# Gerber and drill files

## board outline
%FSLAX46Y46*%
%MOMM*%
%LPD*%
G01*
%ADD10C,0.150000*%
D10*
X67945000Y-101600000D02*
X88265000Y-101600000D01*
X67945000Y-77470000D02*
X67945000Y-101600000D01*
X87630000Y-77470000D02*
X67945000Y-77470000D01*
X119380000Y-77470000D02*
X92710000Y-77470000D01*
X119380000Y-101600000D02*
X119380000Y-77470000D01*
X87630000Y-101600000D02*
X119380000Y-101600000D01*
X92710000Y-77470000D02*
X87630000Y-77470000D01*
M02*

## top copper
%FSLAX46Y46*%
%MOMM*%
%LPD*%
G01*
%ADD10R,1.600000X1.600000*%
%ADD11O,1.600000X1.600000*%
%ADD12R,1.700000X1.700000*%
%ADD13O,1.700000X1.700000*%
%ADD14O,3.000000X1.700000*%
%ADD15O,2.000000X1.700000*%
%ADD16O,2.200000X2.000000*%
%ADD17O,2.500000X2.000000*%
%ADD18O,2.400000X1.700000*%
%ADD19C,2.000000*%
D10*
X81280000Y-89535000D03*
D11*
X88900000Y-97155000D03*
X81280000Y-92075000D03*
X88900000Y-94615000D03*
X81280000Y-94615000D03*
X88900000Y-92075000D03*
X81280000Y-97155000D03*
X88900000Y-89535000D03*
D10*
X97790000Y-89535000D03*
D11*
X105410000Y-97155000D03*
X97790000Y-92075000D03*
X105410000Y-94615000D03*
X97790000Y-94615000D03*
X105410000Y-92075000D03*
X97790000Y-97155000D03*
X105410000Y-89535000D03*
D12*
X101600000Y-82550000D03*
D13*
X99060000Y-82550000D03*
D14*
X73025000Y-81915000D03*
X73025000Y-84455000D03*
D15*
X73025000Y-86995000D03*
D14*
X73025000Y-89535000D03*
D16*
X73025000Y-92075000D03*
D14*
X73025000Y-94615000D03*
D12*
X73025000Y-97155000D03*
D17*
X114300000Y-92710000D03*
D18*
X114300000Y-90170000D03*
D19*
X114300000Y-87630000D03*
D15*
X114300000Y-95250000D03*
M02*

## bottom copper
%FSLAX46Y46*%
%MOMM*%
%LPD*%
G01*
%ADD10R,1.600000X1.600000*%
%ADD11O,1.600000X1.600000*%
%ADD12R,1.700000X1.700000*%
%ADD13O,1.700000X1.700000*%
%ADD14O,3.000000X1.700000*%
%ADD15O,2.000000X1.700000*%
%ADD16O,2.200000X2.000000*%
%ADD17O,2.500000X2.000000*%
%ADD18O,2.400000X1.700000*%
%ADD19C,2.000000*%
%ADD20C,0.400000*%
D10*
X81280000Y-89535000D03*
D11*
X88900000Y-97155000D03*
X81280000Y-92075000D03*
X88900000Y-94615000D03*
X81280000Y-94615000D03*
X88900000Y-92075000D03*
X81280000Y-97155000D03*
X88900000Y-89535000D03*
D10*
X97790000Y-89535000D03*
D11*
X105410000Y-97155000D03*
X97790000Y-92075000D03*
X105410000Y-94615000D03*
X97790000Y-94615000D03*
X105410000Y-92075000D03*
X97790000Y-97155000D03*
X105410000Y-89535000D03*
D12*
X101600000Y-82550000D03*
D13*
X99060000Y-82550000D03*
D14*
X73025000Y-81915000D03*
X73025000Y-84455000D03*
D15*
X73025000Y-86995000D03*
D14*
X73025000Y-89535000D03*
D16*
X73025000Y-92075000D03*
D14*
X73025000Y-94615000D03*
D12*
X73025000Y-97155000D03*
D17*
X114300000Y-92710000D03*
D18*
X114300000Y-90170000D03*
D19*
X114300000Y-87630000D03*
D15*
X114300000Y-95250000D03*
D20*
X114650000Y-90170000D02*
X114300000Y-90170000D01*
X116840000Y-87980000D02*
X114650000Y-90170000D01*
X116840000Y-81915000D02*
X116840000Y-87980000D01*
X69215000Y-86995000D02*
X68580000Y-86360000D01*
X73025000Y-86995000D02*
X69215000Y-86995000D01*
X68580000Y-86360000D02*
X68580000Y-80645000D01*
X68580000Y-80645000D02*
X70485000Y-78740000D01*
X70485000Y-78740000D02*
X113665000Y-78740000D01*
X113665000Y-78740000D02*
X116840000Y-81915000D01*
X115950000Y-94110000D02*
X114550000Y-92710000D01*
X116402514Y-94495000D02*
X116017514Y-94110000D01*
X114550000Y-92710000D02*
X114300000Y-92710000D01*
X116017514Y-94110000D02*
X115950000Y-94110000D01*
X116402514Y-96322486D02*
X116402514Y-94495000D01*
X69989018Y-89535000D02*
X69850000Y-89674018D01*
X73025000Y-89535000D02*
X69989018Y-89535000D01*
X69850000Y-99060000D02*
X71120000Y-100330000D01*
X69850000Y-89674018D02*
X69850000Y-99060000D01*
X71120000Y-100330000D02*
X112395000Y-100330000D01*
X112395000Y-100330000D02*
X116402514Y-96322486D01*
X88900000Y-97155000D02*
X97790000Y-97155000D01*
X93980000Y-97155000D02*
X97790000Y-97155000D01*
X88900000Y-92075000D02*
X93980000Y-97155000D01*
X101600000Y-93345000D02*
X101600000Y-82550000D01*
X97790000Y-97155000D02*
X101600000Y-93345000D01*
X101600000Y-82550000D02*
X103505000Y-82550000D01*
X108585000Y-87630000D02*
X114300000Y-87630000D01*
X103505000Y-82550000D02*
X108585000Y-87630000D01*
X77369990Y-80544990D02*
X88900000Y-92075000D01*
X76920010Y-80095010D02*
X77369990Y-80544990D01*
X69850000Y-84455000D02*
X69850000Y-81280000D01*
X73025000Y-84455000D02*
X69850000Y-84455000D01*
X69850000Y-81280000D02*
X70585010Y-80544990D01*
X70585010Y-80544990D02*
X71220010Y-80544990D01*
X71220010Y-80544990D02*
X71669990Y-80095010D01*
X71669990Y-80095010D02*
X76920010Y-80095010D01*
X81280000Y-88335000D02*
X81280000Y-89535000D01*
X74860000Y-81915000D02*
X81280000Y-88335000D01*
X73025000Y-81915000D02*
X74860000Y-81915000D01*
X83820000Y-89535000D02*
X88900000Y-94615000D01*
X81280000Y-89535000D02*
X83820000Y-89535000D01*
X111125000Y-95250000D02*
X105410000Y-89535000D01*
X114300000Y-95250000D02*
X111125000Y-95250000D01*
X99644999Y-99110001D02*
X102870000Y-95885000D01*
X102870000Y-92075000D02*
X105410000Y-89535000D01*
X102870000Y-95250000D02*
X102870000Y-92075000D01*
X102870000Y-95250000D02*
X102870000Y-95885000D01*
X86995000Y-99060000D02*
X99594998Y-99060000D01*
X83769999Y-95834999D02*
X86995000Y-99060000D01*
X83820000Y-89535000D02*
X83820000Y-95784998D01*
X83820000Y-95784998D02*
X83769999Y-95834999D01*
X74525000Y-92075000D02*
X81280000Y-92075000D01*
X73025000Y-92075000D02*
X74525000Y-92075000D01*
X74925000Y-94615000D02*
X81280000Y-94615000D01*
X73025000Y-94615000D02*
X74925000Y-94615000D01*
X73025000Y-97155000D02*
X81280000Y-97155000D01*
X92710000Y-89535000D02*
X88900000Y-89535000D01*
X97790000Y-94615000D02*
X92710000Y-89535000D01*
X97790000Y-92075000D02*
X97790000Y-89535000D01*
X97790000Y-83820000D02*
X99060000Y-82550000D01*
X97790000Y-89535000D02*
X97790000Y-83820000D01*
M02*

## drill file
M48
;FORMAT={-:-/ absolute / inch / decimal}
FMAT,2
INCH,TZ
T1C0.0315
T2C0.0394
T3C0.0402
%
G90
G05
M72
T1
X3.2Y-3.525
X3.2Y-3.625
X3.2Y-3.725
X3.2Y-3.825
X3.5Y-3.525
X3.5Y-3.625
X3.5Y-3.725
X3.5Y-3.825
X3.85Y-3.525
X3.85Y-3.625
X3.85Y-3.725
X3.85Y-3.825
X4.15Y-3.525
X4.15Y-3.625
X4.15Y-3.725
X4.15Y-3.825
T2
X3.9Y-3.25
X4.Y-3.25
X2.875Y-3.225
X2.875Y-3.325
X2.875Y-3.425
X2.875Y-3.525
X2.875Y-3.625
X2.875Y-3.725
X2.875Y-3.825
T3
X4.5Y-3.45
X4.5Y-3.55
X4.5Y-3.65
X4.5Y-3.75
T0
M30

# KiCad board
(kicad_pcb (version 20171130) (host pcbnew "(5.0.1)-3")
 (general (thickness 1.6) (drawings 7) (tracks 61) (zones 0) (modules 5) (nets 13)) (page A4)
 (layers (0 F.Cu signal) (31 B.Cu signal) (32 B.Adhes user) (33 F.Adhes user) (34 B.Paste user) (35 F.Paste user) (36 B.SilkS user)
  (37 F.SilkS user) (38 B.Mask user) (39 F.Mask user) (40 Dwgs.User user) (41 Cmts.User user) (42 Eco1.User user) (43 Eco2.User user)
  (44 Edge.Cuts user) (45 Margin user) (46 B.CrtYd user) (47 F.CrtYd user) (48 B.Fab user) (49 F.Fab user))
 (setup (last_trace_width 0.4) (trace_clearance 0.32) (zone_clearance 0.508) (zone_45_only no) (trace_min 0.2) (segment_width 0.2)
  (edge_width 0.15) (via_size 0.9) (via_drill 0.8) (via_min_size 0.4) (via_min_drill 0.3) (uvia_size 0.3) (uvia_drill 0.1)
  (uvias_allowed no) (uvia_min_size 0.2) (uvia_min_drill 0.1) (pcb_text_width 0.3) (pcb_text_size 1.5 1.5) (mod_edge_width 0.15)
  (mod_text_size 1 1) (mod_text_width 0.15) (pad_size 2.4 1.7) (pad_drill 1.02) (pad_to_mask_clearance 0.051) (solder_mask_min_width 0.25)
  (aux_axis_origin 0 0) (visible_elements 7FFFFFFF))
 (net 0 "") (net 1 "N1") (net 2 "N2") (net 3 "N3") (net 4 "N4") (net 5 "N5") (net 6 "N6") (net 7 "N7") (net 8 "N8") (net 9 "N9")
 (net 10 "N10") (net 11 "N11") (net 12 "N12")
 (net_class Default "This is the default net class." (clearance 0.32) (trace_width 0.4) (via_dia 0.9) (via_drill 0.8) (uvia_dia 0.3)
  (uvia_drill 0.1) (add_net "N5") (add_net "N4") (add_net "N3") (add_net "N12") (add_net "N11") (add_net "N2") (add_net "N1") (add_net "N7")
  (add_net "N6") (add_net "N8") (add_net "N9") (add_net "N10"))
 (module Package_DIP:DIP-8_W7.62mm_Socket (layer F.Cu) (at 81.28 89.535)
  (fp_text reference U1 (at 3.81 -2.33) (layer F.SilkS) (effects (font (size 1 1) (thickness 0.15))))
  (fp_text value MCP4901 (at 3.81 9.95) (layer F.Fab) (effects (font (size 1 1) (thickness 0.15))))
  (pad 1 thru_hole rect (at 0 0) (size 1.6 1.6) (drill 0.8) (layers *.Cu *.Mask) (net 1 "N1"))
  (pad 5 thru_hole oval (at 7.62 7.62) (size 1.6 1.6) (drill 0.8) (layers *.Cu *.Mask) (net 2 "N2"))
  (pad 2 thru_hole oval (at 0 2.54) (size 1.6 1.6) (drill 0.8) (layers *.Cu *.Mask) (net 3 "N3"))
  (pad 6 thru_hole oval (at 7.62 5.08) (size 1.6 1.6) (drill 0.8) (layers *.Cu *.Mask) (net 1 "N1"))
  (pad 3 thru_hole oval (at 0 5.08) (size 1.6 1.6) (drill 0.8) (layers *.Cu *.Mask) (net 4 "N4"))
  (pad 7 thru_hole oval (at 7.62 2.54) (size 1.6 1.6) (drill 0.8) (layers *.Cu *.Mask) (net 2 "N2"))
  (pad 4 thru_hole oval (at 0 7.62) (size 1.6 1.6) (drill 0.8) (layers *.Cu *.Mask) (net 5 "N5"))
  (pad 8 thru_hole oval (at 7.62 0) (size 1.6 1.6) (drill 0.8) (layers *.Cu *.Mask) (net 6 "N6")))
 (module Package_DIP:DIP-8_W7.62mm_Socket (layer F.Cu) (at 97.79 89.535)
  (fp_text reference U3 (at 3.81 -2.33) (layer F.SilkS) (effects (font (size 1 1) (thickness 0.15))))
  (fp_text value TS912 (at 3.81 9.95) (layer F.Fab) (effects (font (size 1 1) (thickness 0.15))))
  (pad 1 thru_hole rect (at 0 0) (size 1.6 1.6) (drill 0.8) (layers *.Cu *.Mask) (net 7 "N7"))
  (pad 5 thru_hole oval (at 7.62 7.62) (size 1.6 1.6) (drill 0.8) (layers *.Cu *.Mask) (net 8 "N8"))
  (pad 2 thru_hole oval (at 0 2.54) (size 1.6 1.6) (drill 0.8) (layers *.Cu *.Mask) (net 7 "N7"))
  (pad 6 thru_hole oval (at 7.62 5.08) (size 1.6 1.6) (drill 0.8) (layers *.Cu *.Mask) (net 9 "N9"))
  (pad 3 thru_hole oval (at 0 5.08) (size 1.6 1.6) (drill 0.8) (layers *.Cu *.Mask) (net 6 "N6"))
  (pad 7 thru_hole oval (at 7.62 2.54) (size 1.6 1.6) (drill 0.8) (layers *.Cu *.Mask) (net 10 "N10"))
  (pad 4 thru_hole oval (at 0 7.62) (size 1.6 1.6) (drill 0.8) (layers *.Cu *.Mask) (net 2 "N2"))
  (pad 8 thru_hole oval (at 7.62 0) (size 1.6 1.6) (drill 0.8) (layers *.Cu *.Mask) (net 1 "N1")))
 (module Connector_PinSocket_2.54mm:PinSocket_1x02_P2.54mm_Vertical (layer F.Cu) (at 101.6 82.55 270)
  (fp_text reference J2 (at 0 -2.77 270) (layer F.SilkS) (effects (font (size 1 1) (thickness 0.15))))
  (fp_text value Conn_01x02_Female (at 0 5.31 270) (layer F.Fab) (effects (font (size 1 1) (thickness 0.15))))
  (pad 1 thru_hole rect (at 0 0 270) (size 1.7 1.7) (drill 1) (layers *.Cu *.Mask) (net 2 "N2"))
  (pad 2 thru_hole oval (at 0 2.54 270) (size 1.7 1.7) (drill 1) (layers *.Cu *.Mask) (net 7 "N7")))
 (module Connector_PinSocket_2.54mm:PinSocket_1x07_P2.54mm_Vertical (layer F.Cu) (at 73.025 97.155 180)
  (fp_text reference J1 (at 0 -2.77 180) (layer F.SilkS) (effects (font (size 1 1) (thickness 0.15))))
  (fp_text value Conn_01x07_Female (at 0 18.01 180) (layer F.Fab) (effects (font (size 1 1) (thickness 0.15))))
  (pad 7 thru_hole oval (at 0 15.24 180) (size 3 1.7) (drill 1) (layers *.Cu *.Mask) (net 1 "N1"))
  (pad 6 thru_hole oval (at 0 12.7 180) (size 3 1.7) (drill 1) (layers *.Cu *.Mask) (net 2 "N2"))
  (pad 5 thru_hole oval (at 0 10.16 180) (size 2 1.7) (drill 1) (layers *.Cu *.Mask) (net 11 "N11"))
  (pad 4 thru_hole oval (at 0 7.62 180) (size 3 1.7) (drill 1) (layers *.Cu *.Mask) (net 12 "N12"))
  (pad 3 thru_hole oval (at 0 5.08 180) (size 2.2 2) (drill 1) (layers *.Cu *.Mask) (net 3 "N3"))
  (pad 2 thru_hole oval (at 0 2.54 180) (size 3 1.7) (drill 1) (layers *.Cu *.Mask) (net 4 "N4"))
  (pad 1 thru_hole rect (at 0 0 180) (size 1.7 1.7) (drill 1) (layers *.Cu *.Mask) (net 5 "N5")))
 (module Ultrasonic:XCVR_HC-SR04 (layer F.Cu) (at 114.3 91.44 90)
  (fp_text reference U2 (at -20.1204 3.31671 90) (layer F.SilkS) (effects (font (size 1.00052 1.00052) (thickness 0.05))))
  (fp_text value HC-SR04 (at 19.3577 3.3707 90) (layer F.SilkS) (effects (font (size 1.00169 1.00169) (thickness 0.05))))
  (pad 2 thru_hole oval (at -1.27 0 90) (size 2 2.5) (drill 1.02) (layers *.Cu *.Mask) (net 12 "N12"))
  (pad 3 thru_hole oval (at 1.27 0 180) (size 2.4 1.7) (drill 1.02) (layers *.Cu *.Mask) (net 11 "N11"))
  (pad 4 thru_hole circle (at 3.81 0 90) (size 2 2) (drill 1.02) (layers *.Cu *.Mask) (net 2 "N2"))
  (pad 1 thru_hole oval (at -3.81 0 180) (size 2 1.7) (drill 1.02) (layers *.Cu *.Mask) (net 1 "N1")))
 (gr_line (start 67.945 101.6) (end 88.265 101.6) (layer Edge.Cuts) (width 0.15))
 (gr_line (start 67.945 77.47) (end 67.945 101.6) (layer Edge.Cuts) (width 0.15))
 (gr_line (start 87.63 77.47) (end 67.945 77.47) (layer Edge.Cuts) (width 0.15))
 (gr_line (start 119.38 77.47) (end 92.71 77.47) (layer Edge.Cuts) (width 0.15))
 (gr_line (start 119.38 101.6) (end 119.38 77.47) (layer Edge.Cuts) (width 0.15))
 (gr_line (start 87.63 101.6) (end 119.38 101.6) (layer Edge.Cuts) (width 0.15))
 (gr_line (start 92.71 77.47) (end 87.63 77.47) (layer Edge.Cuts) (width 0.15))
 (segment (start 114.65 90.17) (end 114.3 90.17) (width 0.4) (layer B.Cu) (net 11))
 (segment (start 116.84 87.98) (end 114.65 90.17) (width 0.4) (layer B.Cu) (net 11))
 (segment (start 116.84 81.915) (end 116.84 87.98) (width 0.4) (layer B.Cu) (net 11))
 (segment (start 69.215 86.995) (end 68.58 86.36) (width 0.4) (layer B.Cu) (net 11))
 (segment (start 73.025 86.995) (end 69.215 86.995) (width 0.4) (layer B.Cu) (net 11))
 (segment (start 68.58 86.36) (end 68.58 80.645) (width 0.4) (layer B.Cu) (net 11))
 (segment (start 68.58 80.645) (end 70.485 78.74) (width 0.4) (layer B.Cu) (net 11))
 (segment (start 70.485 78.74) (end 113.665 78.74) (width 0.4) (layer B.Cu) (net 11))
 (segment (start 113.665 78.74) (end 116.84 81.915) (width 0.4) (layer B.Cu) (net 11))
 (segment (start 115.95 94.11) (end 114.55 92.71) (width 0.4) (layer B.Cu) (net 12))
 (segment (start 116.402514 94.495) (end 116.017514 94.11) (width 0.4) (layer B.Cu) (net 12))
 (segment (start 114.55 92.71) (end 114.3 92.71) (width 0.4) (layer B.Cu) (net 12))
 (segment (start 116.017514 94.11) (end 115.95 94.11) (width 0.4) (layer B.Cu) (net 12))
 (segment (start 116.402514 96.322486) (end 116.402514 94.495) (width 0.4) (layer B.Cu) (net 12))
 (segment (start 69.989018 89.535) (end 69.85 89.674018) (width 0.4) (layer B.Cu) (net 12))
 (segment (start 73.025 89.535) (end 69.989018 89.535) (width 0.4) (layer B.Cu) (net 12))
 (segment (start 69.85 99.06) (end 71.12 100.33) (width 0.4) (layer B.Cu) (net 12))
 (segment (start 69.85 89.674018) (end 69.85 99.06) (width 0.4) (layer B.Cu) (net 12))
 (segment (start 71.12 100.33) (end 112.395 100.33) (width 0.4) (layer B.Cu) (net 12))
 (segment (start 112.395 100.33) (end 116.402514 96.322486) (width 0.4) (layer B.Cu) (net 12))
 (segment (start 88.9 97.155) (end 97.79 97.155) (width 0.4) (layer B.Cu) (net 2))
 (segment (start 93.98 97.155) (end 97.79 97.155) (width 0.4) (layer B.Cu) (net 2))
 (segment (start 88.9 92.075) (end 93.98 97.155) (width 0.4) (layer B.Cu) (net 2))
 (segment (start 101.6 93.345) (end 101.6 82.55) (width 0.4) (layer B.Cu) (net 2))
 (segment (start 97.79 97.155) (end 101.6 93.345) (width 0.4) (layer B.Cu) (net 2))
 (segment (start 101.6 82.55) (end 103.505 82.55) (width 0.4) (layer B.Cu) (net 2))
 (segment (start 108.585 87.63) (end 114.3 87.63) (width 0.4) (layer B.Cu) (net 2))
 (segment (start 103.505 82.55) (end 108.585 87.63) (width 0.4) (layer B.Cu) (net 2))
 (segment (start 77.36999 80.54499) (end 88.9 92.075) (width 0.4) (layer B.Cu) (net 2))
 (segment (start 76.92001 80.09501) (end 77.36999 80.54499) (width 0.4) (layer B.Cu) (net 2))
 (segment (start 69.85 84.455) (end 69.85 81.28) (width 0.4) (layer B.Cu) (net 2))
 (segment (start 73.025 84.455) (end 69.85 84.455) (width 0.4) (layer B.Cu) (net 2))
 (segment (start 69.85 81.28) (end 70.58501 80.54499) (width 0.4) (layer B.Cu) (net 2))
 (segment (start 70.58501 80.54499) (end 71.22001 80.54499) (width 0.4) (layer B.Cu) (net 2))
 (segment (start 71.22001 80.54499) (end 71.66999 80.09501) (width 0.4) (layer B.Cu) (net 2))
 (segment (start 71.66999 80.09501) (end 76.92001 80.09501) (width 0.4) (layer B.Cu) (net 2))
 (segment (start 81.28 88.335) (end 81.28 89.535) (width 0.4) (layer B.Cu) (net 1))
 (segment (start 74.86 81.915) (end 81.28 88.335) (width 0.4) (layer B.Cu) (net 1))
 (segment (start 73.025 81.915) (end 74.86 81.915) (width 0.4) (layer B.Cu) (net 1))
 (segment (start 83.82 89.535) (end 88.9 94.615) (width 0.4) (layer B.Cu) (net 1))
 (segment (start 81.28 89.535) (end 83.82 89.535) (width 0.4) (layer B.Cu) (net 1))
 (segment (start 111.125 95.25) (end 105.41 89.535) (width 0.4) (layer B.Cu) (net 1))
 (segment (start 114.3 95.25) (end 111.125 95.25) (width 0.4) (layer B.Cu) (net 1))
 (segment (start 99.644999 99.110001) (end 102.87 95.885) (width 0.4) (layer B.Cu) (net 1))
 (segment (start 102.87 92.075) (end 105.41 89.535) (width 0.4) (layer B.Cu) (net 1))
 (segment (start 102.87 95.25) (end 102.87 92.075) (width 0.4) (layer B.Cu) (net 1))
 (segment (start 102.87 95.25) (end 102.87 95.885) (width 0.4) (layer B.Cu) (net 1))
 (segment (start 86.995 99.06) (end 99.594998 99.06) (width 0.4) (layer B.Cu) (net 1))
 (segment (start 83.769999 95.834999) (end 86.995 99.06) (width 0.4) (layer B.Cu) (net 1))
 (segment (start 83.82 89.535) (end 83.82 95.784998) (width 0.4) (layer B.Cu) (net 1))
 (segment (start 83.82 95.784998) (end 83.769999 95.834999) (width 0.4) (layer B.Cu) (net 1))
 (segment (start 74.525 92.075) (end 81.28 92.075) (width 0.4) (layer B.Cu) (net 3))
 (segment (start 73.025 92.075) (end 74.525 92.075) (width 0.4) (layer B.Cu) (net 3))
 (segment (start 74.925 94.615) (end 81.28 94.615) (width 0.4) (layer B.Cu) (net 4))
 (segment (start 73.025 94.615) (end 74.925 94.615) (width 0.4) (layer B.Cu) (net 4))
 (segment (start 73.025 97.155) (end 81.28 97.155) (width 0.4) (layer B.Cu) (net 5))
 (segment (start 92.71 89.535) (end 88.9 89.535) (width 0.4) (layer B.Cu) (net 6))
 (segment (start 97.79 94.615) (end 92.71 89.535) (width 0.4) (layer B.Cu) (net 6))
 (segment (start 97.79 92.075) (end 97.79 89.535) (width 0.4) (layer B.Cu) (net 7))
 (segment (start 97.79 83.82) (end 99.06 82.55) (width 0.4) (layer B.Cu) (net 7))
 (segment (start 97.79 89.535) (end 97.79 83.82) (width 0.4) (layer B.Cu) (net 7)))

